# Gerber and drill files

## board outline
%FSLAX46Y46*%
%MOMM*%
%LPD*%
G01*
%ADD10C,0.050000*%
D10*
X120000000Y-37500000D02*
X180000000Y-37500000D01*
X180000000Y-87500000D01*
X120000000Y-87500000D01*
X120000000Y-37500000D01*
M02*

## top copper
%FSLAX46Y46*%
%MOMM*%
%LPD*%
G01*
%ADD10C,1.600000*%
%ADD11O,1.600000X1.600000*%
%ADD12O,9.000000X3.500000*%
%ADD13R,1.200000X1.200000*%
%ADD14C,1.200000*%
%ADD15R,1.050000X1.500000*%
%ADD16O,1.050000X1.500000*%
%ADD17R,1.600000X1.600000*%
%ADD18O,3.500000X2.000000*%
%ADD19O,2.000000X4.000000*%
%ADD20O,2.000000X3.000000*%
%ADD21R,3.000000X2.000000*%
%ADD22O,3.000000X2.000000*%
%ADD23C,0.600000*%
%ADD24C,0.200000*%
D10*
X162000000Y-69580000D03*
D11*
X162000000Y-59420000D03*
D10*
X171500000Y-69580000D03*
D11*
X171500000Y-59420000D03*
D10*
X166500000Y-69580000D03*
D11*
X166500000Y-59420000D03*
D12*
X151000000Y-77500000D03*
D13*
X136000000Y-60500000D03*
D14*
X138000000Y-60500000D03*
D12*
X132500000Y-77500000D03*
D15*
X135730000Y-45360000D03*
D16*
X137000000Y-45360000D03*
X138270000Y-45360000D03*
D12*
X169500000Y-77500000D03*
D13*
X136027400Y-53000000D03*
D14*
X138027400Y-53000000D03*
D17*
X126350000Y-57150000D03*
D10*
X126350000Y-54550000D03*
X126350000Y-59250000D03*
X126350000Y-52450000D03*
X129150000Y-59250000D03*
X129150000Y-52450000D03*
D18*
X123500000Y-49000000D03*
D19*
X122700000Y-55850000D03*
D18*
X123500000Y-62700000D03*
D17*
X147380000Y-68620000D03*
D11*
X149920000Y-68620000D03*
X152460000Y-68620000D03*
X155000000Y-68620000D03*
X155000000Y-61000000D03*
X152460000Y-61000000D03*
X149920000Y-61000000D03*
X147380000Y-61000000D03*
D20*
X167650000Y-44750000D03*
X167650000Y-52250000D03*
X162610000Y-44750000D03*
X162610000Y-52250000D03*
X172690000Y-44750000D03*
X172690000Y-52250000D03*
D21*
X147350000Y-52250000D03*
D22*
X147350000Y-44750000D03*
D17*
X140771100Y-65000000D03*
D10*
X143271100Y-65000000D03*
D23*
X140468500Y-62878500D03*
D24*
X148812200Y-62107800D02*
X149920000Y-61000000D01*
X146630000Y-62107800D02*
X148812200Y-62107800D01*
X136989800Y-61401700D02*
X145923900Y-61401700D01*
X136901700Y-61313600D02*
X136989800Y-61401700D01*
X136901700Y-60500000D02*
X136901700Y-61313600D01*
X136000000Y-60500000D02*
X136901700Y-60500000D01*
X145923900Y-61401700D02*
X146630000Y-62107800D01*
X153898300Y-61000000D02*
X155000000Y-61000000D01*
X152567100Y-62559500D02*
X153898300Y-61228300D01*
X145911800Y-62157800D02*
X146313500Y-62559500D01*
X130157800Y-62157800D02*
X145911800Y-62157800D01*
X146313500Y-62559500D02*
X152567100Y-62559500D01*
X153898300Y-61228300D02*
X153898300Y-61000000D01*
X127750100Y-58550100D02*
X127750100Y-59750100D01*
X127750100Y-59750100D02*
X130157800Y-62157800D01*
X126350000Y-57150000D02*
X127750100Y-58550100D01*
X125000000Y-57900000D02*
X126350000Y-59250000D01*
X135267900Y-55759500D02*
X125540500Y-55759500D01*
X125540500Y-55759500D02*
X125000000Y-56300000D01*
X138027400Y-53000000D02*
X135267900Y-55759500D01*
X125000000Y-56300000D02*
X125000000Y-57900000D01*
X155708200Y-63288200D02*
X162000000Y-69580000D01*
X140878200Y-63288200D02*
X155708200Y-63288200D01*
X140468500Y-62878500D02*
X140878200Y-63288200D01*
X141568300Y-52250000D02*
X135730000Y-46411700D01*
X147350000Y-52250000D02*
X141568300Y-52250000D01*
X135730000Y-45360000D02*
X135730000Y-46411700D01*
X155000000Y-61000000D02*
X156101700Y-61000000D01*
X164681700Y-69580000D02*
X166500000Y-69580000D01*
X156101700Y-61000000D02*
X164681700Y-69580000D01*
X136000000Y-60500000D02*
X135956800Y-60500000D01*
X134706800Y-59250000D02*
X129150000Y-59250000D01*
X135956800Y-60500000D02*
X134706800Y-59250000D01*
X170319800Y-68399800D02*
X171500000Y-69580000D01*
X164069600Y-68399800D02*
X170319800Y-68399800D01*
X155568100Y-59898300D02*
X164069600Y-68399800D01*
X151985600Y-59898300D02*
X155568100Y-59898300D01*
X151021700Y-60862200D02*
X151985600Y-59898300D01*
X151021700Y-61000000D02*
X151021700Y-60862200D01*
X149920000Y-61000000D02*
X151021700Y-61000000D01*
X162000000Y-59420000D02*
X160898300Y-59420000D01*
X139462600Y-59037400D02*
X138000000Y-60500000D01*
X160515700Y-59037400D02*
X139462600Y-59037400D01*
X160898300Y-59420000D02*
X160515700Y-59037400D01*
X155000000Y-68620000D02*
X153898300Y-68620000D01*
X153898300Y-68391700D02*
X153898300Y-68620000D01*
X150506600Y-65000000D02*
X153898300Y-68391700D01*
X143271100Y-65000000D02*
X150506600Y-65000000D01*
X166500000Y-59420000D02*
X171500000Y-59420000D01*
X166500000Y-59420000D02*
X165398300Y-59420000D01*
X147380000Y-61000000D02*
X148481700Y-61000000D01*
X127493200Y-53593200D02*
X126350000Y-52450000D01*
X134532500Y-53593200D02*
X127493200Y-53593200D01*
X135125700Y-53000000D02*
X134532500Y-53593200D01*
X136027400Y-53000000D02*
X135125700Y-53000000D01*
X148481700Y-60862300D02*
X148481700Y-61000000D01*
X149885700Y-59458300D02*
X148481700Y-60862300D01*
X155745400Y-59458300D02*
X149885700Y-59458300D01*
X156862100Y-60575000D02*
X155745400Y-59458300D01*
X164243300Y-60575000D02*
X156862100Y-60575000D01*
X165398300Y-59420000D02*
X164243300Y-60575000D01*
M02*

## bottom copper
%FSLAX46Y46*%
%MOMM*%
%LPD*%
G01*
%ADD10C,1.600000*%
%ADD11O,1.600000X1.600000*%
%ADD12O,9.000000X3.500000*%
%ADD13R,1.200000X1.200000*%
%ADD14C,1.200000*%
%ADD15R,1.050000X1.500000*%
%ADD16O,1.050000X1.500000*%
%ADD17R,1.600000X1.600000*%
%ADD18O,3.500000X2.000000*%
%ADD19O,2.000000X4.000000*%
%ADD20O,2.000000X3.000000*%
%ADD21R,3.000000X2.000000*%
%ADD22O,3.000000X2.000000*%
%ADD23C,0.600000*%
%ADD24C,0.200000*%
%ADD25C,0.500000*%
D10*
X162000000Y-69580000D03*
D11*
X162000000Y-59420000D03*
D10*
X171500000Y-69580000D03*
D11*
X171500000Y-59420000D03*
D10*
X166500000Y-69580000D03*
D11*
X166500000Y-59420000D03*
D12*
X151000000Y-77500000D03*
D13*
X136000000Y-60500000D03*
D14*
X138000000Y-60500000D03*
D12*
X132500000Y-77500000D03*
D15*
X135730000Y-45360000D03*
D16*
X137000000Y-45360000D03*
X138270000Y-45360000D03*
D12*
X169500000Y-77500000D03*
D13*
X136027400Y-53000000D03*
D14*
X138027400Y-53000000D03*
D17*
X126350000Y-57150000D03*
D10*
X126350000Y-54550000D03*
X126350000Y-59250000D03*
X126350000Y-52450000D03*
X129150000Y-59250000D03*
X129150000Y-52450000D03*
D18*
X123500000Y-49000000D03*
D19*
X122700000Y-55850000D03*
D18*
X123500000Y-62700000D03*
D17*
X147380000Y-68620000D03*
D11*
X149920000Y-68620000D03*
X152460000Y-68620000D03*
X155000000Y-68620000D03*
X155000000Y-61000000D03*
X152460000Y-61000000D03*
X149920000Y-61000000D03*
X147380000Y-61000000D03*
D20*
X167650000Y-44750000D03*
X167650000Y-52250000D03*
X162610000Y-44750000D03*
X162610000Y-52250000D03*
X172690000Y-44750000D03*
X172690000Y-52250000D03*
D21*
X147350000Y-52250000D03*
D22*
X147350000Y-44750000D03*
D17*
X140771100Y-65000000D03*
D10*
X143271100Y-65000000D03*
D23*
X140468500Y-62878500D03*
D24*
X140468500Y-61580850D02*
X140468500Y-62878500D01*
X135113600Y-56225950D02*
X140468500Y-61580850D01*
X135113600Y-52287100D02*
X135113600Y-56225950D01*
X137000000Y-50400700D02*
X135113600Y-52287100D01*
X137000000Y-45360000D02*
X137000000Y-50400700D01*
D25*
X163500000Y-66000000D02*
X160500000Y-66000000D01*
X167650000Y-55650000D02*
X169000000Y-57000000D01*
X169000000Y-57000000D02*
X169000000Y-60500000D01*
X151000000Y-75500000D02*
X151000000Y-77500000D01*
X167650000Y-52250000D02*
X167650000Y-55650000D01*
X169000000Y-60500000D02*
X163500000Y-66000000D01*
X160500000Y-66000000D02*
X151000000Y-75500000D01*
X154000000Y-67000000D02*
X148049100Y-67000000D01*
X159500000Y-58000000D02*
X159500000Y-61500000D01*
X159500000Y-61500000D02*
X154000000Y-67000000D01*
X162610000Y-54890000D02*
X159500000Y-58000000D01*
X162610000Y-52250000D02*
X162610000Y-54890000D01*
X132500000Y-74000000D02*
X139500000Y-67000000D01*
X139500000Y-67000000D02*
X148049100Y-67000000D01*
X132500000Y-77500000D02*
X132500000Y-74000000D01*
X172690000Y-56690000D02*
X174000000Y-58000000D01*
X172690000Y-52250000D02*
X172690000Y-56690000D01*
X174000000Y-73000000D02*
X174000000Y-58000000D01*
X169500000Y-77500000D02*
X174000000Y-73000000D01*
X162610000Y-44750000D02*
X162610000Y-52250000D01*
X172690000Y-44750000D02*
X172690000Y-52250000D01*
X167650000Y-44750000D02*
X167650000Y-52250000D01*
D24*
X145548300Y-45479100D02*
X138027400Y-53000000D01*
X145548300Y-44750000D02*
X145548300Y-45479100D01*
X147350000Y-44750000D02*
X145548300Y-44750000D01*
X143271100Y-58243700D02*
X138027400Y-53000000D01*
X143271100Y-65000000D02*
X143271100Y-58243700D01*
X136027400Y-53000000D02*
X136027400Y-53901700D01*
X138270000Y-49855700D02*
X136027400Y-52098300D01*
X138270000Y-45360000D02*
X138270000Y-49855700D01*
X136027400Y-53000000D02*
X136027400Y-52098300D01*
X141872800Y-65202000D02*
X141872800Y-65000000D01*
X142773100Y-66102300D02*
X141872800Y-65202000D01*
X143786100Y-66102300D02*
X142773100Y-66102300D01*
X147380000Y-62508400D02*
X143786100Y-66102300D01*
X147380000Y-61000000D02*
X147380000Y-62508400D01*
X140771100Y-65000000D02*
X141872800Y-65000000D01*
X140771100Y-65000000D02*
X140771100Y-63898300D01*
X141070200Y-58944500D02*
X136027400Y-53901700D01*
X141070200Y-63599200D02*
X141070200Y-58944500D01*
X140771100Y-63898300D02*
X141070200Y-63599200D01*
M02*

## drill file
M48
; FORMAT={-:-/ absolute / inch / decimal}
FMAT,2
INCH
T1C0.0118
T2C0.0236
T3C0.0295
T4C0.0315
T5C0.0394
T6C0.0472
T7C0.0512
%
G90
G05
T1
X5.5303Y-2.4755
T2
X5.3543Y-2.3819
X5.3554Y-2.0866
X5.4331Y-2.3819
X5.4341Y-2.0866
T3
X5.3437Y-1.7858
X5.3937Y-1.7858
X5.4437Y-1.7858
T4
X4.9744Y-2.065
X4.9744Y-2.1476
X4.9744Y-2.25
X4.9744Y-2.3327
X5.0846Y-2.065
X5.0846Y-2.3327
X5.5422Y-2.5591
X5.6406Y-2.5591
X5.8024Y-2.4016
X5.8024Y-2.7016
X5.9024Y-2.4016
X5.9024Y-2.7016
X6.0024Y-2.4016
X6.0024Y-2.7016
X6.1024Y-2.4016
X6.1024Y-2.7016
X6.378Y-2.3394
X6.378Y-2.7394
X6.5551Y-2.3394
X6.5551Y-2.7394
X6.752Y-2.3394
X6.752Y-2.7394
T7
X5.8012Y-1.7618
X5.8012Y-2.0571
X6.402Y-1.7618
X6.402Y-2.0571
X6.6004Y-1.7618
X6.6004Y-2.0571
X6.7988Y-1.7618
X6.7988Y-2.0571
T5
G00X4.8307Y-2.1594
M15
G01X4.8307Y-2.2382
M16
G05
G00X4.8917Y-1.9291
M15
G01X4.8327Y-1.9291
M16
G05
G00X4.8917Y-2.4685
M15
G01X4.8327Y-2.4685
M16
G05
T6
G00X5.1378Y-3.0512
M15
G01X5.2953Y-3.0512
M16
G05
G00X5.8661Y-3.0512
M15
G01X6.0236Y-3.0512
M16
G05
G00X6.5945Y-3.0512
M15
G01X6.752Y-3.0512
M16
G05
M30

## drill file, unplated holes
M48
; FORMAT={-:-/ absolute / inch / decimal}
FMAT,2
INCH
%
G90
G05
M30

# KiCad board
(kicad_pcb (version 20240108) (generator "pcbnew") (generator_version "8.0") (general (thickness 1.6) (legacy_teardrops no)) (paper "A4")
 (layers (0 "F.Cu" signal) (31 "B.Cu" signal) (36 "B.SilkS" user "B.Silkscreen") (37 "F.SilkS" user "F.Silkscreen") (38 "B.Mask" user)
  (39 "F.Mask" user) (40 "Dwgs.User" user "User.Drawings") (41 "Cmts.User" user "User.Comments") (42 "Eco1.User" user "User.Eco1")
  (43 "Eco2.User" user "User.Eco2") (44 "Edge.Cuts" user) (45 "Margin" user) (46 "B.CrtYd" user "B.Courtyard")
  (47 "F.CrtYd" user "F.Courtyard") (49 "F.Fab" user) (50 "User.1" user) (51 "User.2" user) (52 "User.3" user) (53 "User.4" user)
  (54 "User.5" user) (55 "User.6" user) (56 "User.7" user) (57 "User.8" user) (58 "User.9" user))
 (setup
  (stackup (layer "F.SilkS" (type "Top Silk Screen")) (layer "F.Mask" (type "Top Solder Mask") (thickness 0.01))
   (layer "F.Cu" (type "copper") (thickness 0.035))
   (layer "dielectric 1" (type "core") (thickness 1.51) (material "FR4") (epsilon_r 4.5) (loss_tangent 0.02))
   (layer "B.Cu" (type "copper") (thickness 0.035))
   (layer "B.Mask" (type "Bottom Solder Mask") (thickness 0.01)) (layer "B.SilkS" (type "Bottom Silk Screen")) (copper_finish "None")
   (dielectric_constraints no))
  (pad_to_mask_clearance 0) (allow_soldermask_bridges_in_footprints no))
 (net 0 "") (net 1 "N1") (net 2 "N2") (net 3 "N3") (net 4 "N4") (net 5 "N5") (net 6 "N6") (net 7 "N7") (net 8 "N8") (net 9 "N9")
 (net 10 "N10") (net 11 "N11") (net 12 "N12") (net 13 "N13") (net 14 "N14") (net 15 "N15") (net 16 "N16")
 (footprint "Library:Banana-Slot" (layer "F.Cu") (at 151 81.5)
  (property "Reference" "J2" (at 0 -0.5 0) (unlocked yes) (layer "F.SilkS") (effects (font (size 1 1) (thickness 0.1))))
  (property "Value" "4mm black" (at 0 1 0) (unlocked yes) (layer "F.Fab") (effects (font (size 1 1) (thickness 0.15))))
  (pad "1" thru_hole oval (at 0 -4) (size 9 3.5) (drill oval 5.2 1.2) (layers "*.Cu" "*.Mask") (remove_unused_layers no) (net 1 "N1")))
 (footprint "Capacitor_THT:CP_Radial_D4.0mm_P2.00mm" (layer "F.Cu") (at 136 60.5)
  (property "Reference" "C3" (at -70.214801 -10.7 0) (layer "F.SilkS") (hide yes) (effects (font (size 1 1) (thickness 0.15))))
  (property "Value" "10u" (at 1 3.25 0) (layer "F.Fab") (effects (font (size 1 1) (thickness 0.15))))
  (pad "1" thru_hole rect (at 0 0) (size 1.2 1.2) (drill 0.6) (layers "*.Cu" "*.Mask") (remove_unused_layers no) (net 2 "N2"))
  (pad "2" thru_hole circle (at 2 0) (size 1.2 1.2) (drill 0.6) (layers "*.Cu" "*.Mask") (remove_unused_layers no) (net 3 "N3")))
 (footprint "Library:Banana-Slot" (layer "F.Cu") (at 132.5 81.5)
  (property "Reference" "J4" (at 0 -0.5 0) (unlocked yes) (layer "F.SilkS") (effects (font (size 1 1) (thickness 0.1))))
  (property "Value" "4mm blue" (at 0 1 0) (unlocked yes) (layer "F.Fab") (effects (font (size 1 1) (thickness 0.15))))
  (pad "1" thru_hole oval (at 0 -4) (size 9 3.5) (drill oval 5.2 1.2) (layers "*.Cu" "*.Mask") (remove_unused_layers no) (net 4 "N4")))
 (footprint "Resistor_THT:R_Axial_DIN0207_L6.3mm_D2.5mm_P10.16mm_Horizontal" (layer "F.Cu") (at 171.5 69.58 90)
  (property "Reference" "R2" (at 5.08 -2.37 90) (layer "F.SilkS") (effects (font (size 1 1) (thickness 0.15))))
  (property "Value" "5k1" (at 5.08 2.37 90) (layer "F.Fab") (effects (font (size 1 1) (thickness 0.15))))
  (pad "1" thru_hole circle (at 0 0 90) (size 1.6 1.6) (drill 0.8) (layers "*.Cu" "*.Mask") (remove_unused_layers no) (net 2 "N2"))
  (pad "2" thru_hole oval (at 10.16 0 90) (size 1.6 1.6) (drill 0.8) (layers "*.Cu" "*.Mask") (remove_unused_layers no) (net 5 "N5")))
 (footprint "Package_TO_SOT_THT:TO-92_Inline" (layer "F.Cu") (at 135.73 45.36)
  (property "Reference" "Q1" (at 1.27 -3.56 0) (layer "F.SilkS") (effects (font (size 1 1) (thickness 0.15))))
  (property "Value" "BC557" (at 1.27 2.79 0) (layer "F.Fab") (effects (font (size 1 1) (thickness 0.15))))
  (pad "1" thru_hole rect (at 0 0) (size 1.05 1.5) (drill 0.75) (layers "*.Cu" "*.Mask") (remove_unused_layers no) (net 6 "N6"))
  (pad "2" thru_hole oval (at 1.27 0) (size 1.05 1.5) (drill 0.75) (layers "*.Cu" "*.Mask") (remove_unused_layers no) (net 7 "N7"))
  (pad "3" thru_hole oval (at 2.54 0) (size 1.05 1.5) (drill 0.75) (layers "*.Cu" "*.Mask") (remove_unused_layers no) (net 5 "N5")))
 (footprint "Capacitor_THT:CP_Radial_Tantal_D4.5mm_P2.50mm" (layer "F.Cu") (at 140.7711 65)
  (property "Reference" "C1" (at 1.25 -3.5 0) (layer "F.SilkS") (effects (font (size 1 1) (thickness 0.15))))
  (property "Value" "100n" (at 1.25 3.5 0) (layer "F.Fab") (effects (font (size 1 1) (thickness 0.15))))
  (pad "1" thru_hole rect (at 0 0) (size 1.6 1.6) (drill 0.8) (layers "*.Cu" "*.Mask") (remove_unused_layers no) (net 5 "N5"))
  (pad "2" thru_hole circle (at 2.5 0) (size 1.6 1.6) (drill 0.8) (layers "*.Cu" "*.Mask") (remove_unused_layers no) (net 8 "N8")))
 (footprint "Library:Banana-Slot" (layer "F.Cu") (at 169.5 81.5)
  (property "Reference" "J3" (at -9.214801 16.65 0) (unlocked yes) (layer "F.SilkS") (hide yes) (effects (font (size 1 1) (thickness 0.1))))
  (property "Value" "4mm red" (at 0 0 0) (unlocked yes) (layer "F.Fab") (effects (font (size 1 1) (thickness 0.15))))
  (pad "1" thru_hole oval (at 0 -4) (size 9 3.5) (drill oval 5.2 1.2) (layers "*.Cu" "*.Mask") (remove_unused_layers no) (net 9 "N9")))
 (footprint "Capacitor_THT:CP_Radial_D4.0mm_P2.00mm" (layer "F.Cu") (at 136.0274 53)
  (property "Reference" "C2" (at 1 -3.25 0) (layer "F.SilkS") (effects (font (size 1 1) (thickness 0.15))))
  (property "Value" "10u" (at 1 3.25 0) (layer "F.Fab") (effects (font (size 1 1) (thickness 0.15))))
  (pad "1" thru_hole rect (at 0 0) (size 1.2 1.2) (drill 0.6) (layers "*.Cu" "*.Mask") (remove_unused_layers no) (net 5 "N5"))
  (pad "2" thru_hole circle (at 2 0) (size 1.2 1.2) (drill 0.6) (layers "*.Cu" "*.Mask") (remove_unused_layers no) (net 8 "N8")))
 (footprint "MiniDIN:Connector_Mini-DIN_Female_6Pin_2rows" (layer "F.Cu") (at 126.35 57.15 -90)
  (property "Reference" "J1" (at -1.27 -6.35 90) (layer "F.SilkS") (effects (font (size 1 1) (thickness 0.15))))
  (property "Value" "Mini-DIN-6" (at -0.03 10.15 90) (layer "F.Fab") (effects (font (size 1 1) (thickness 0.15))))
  (pad "1" thru_hole rect (at 0 0 270) (size 1.6 1.6) (drill 0.8) (layers "*.Cu" "*.Mask") (remove_unused_layers no) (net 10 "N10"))
  (pad "2" thru_hole circle (at -2.6 0 270) (size 1.6 1.6) (drill 0.8) (layers "*.Cu" "*.Mask") (remove_unused_layers no) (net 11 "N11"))
  (pad "3" thru_hole circle (at 2.1 0 270) (size 1.6 1.6) (drill 0.8) (layers "*.Cu" "*.Mask") (remove_unused_layers no) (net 8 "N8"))
  (pad "4" thru_hole circle (at -4.7 0 270) (size 1.6 1.6) (drill 0.8) (layers "*.Cu" "*.Mask") (remove_unused_layers no) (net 5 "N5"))
  (pad "5" thru_hole circle (at 2.1 -2.8 270) (size 1.6 1.6) (drill 0.8) (layers "*.Cu" "*.Mask") (remove_unused_layers no) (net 2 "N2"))
  (pad "6" thru_hole circle (at -4.7 -2.8 270) (size 1.6 1.6) (drill 0.8) (layers "*.Cu" "*.Mask") (remove_unused_layers no) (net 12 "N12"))
  (pad "7" thru_hole oval (at -8.15 2.85 270) (size 2 3.5) (drill oval 1 2.5) (layers "*.Cu" "*.Mask") (remove_unused_layers no))
  (pad "7" thru_hole oval (at -1.3 3.65 270) (size 4 2) (drill oval 3 1) (layers "*.Cu" "*.Mask") (remove_unused_layers no))
  (pad "7" thru_hole oval (at 5.55 2.85 270) (size 2 3.5) (drill oval 1 2.5) (layers "*.Cu" "*.Mask") (remove_unused_layers no)))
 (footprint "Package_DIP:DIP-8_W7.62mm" (layer "F.Cu") (at 147.38 68.62 90)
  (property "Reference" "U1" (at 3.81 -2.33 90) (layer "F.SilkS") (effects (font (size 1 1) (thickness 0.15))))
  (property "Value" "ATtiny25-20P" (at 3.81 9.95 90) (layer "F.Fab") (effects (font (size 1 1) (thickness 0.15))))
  (pad "1" thru_hole rect (at 0 0 90) (size 1.6 1.6) (drill 0.8) (layers "*.Cu" "*.Mask") (remove_unused_layers no) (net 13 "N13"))
  (pad "2" thru_hole oval (at 0 2.54 90) (size 1.6 1.6) (drill 0.8) (layers "*.Cu" "*.Mask") (remove_unused_layers no) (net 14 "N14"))
  (pad "3" thru_hole oval (at 0 5.08 90) (size 1.6 1.6) (drill 0.8) (layers "*.Cu" "*.Mask") (remove_unused_layers no) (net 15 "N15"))
  (pad "4" thru_hole oval (at 0 7.62 90) (size 1.6 1.6) (drill 0.8) (layers "*.Cu" "*.Mask") (remove_unused_layers no) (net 8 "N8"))
  (pad "5" thru_hole oval (at 7.62 7.62 90) (size 1.6 1.6) (drill 0.8) (layers "*.Cu" "*.Mask") (remove_unused_layers no) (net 10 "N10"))
  (pad "6" thru_hole oval (at 7.62 5.08 90) (size 1.6 1.6) (drill 0.8) (layers "*.Cu" "*.Mask") (remove_unused_layers no) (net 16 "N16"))
  (pad "7" thru_hole oval (at 7.62 2.54 90) (size 1.6 1.6) (drill 0.8) (layers "*.Cu" "*.Mask") (remove_unused_layers no) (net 2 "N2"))
  (pad "8" thru_hole oval (at 7.62 0 90) (size 1.6 1.6) (drill 0.8) (layers "*.Cu" "*.Mask") (remove_unused_layers no) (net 5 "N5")))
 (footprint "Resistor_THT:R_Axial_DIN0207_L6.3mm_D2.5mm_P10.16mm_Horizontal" (layer "F.Cu") (at 162 69.58 90)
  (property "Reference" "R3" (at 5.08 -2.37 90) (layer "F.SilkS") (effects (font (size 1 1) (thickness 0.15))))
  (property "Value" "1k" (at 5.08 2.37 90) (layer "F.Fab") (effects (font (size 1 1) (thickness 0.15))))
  (pad "1" thru_hole circle (at 0 0 90) (size 1.6 1.6) (drill 0.8) (layers "*.Cu" "*.Mask") (remove_unused_layers no) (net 7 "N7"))
  (pad "2" thru_hole oval (at 10.16 0 90) (size 1.6 1.6) (drill 0.8) (layers "*.Cu" "*.Mask") (remove_unused_layers no) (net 3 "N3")))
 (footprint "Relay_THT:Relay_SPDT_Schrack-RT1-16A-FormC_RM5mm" (layer "F.Cu") (at 147.35 52.25)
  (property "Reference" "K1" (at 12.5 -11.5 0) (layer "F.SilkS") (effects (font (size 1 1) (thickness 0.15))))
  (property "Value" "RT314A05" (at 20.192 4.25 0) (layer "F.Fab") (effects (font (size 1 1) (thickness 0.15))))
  (pad "11" thru_hole oval (at 20.3 -7.5 180) (size 2 3) (drill 1.3) (layers "*.Cu" "*.Mask") (remove_unused_layers no) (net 1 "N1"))
  (pad "11" thru_hole oval (at 20.3 0 180) (size 2 3) (drill 1.3) (layers "*.Cu" "*.Mask") (remove_unused_layers no) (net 1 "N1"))
  (pad "12" thru_hole oval (at 15.26 -7.5 180) (size 2 3) (drill 1.3) (layers "*.Cu" "*.Mask") (remove_unused_layers no) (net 4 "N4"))
  (pad "12" thru_hole oval (at 15.26 0 180) (size 2 3) (drill 1.3) (layers "*.Cu" "*.Mask") (remove_unused_layers no) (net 4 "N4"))
  (pad "14" thru_hole oval (at 25.34 -7.5 180) (size 2 3) (drill 1.3) (layers "*.Cu" "*.Mask") (remove_unused_layers no) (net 9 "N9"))
  (pad "14" thru_hole oval (at 25.34 0 180) (size 2 3) (drill 1.3) (layers "*.Cu" "*.Mask") (remove_unused_layers no) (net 9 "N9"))
  (pad "A1" thru_hole rect (at 0 0 180) (size 3 2) (drill 1.3) (layers "*.Cu" "*.Mask") (remove_unused_layers no) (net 6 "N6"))
  (pad "A2" thru_hole oval (at 0 -7.5 180) (size 3 2) (drill 1.3) (layers "*.Cu" "*.Mask") (remove_unused_layers no) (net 8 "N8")))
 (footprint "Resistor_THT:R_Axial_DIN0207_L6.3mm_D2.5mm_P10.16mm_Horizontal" (layer "F.Cu") (at 166.5 69.58 90)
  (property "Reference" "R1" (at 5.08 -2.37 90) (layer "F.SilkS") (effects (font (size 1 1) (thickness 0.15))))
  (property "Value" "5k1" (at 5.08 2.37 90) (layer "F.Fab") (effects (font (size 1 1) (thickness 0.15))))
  (pad "1" thru_hole circle (at 0 0 90) (size 1.6 1.6) (drill 0.8) (layers "*.Cu" "*.Mask") (remove_unused_layers no) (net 10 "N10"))
  (pad "2" thru_hole oval (at 10.16 0 90) (size 1.6 1.6) (drill 0.8) (layers "*.Cu" "*.Mask") (remove_unused_layers no) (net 5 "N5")))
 (gr_rect (start 120 37.5) (end 180 87.5) (stroke (width 0.05) (type default)) (fill none) (layer "Edge.Cuts"))
 (segment (start 149.8857 59.4583) (end 148.4817 60.8623) (width 0.2) (layer "F.Cu") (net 5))
 (segment (start 136.0274 53) (end 135.1257 53) (width 0.2) (layer "F.Cu") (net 5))
 (segment (start 155.7454 59.4583) (end 149.8857 59.4583) (width 0.2) (layer "F.Cu") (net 5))
 (segment (start 134.5325 53.5932) (end 127.4932 53.5932) (width 0.2) (layer "F.Cu") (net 5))
 (segment (start 164.2433 60.575) (end 156.8621 60.575) (width 0.2) (layer "F.Cu") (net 5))
 (segment (start 148.4817 60.8623) (end 148.4817 61) (width 0.2) (layer "F.Cu") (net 5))
 (segment (start 165.3983 59.42) (end 164.2433 60.575) (width 0.2) (layer "F.Cu") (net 5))
 (segment (start 135.1257 53) (end 134.5325 53.5932) (width 0.2) (layer "F.Cu") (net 5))
 (segment (start 166.5 59.42) (end 171.5 59.42) (width 0.2) (layer "F.Cu") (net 5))
 (segment (start 147.38 61) (end 148.4817 61) (width 0.2) (layer "F.Cu") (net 5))
 (segment (start 156.8621 60.575) (end 155.7454 59.4583) (width 0.2) (layer "F.Cu") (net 5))
 (segment (start 166.5 59.42) (end 165.3983 59.42) (width 0.2) (layer "F.Cu") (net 5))
 (segment (start 127.4932 53.5932) (end 126.35 52.45) (width 0.2) (layer "F.Cu") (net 5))
 (segment (start 142.7731 66.1023) (end 141.8728 65.202) (width 0.2) (layer "B.Cu") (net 5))
 (segment (start 140.7711 63.8983) (end 141.0702 63.5992) (width 0.2) (layer "B.Cu") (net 5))
 (segment (start 138.27 49.8557) (end 136.0274 52.0983) (width 0.2) (layer "B.Cu") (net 5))
 (segment (start 136.0274 53) (end 136.0274 53.9017) (width 0.2) (layer "B.Cu") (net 5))
 (segment (start 141.8728 65.202) (end 141.8728 65) (width 0.2) (layer "B.Cu") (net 5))
 (segment (start 147.38 62.5084) (end 143.7861 66.1023) (width 0.2) (layer "B.Cu") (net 5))
 (segment (start 140.7711 65) (end 141.8728 65) (width 0.2) (layer "B.Cu") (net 5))
 (segment (start 143.7861 66.1023) (end 142.7731 66.1023) (width 0.2) (layer "B.Cu") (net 5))
 (segment (start 147.38 61) (end 147.38 62.5084) (width 0.2) (layer "B.Cu") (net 5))
 (segment (start 136.0274 53) (end 136.0274 52.0983) (width 0.2) (layer "B.Cu") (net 5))
 (segment (start 140.7711 65) (end 140.7711 63.8983) (width 0.2) (layer "B.Cu") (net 5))
 (segment (start 141.0702 58.9445) (end 136.0274 53.9017) (width 0.2) (layer "B.Cu") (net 5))
 (segment (start 138.27 45.36) (end 138.27 49.8557) (width 0.2) (layer "B.Cu") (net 5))
 (segment (start 141.0702 63.5992) (end 141.0702 58.9445) (width 0.2) (layer "B.Cu") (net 5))
 (segment (start 143.2711 65) (end 150.5066 65) (width 0.2) (layer "F.Cu") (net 8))
 (segment (start 150.5066 65) (end 153.8983 68.3917) (width 0.2) (layer "F.Cu") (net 8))
 (segment (start 153.8983 68.3917) (end 153.8983 68.62) (width 0.2) (layer "F.Cu") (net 8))
 (segment (start 138.0274 53) (end 135.2679 55.7595) (width 0.2) (layer "F.Cu") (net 8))
 (segment (start 135.2679 55.7595) (end 125.5405 55.7595) (width 0.2) (layer "F.Cu") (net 8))
 (segment (start 125.5405 55.7595) (end 125 56.3) (width 0.2) (layer "F.Cu") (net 8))
 (segment (start 155 68.62) (end 153.8983 68.62) (width 0.2) (layer "F.Cu") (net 8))
 (segment (start 125 56.3) (end 125 57.9) (width 0.2) (layer "F.Cu") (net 8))
 (segment (start 125 57.9) (end 126.35 59.25) (width 0.2) (layer "F.Cu") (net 8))
 (segment (start 143.2711 65) (end 143.2711 58.2437) (width 0.2) (layer "B.Cu") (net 8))
 (segment (start 145.5483 45.4791) (end 138.0274 53) (width 0.2) (layer "B.Cu") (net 8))
 (segment (start 147.35 44.75) (end 145.5483 44.75) (width 0.2) (layer "B.Cu") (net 8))
 (segment (start 145.5483 44.75) (end 145.5483 45.4791) (width 0.2) (layer "B.Cu") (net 8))
 (segment (start 143.2711 58.2437) (end 138.0274 53) (width 0.2) (layer "B.Cu") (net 8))
 (segment (start 139.4626 59.0374) (end 138 60.5) (width 0.2) (layer "F.Cu") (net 3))
 (segment (start 160.8983 59.42) (end 160.5157 59.0374) (width 0.2) (layer "F.Cu") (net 3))
 (segment (start 162 59.42) (end 160.8983 59.42) (width 0.2) (layer "F.Cu") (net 3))
 (segment (start 160.5157 59.0374) (end 139.4626 59.0374) (width 0.2) (layer "F.Cu") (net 3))
 (segment (start 151.9856 59.8983) (end 155.5681 59.8983) (width 0.2) (layer "F.Cu") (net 2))
 (segment (start 136.9017 61.3136) (end 136.9898 61.4017) (width 0.2) (layer "F.Cu") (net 2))
 (segment (start 151.0217 61) (end 151.0217 60.8622) (width 0.2) (layer "F.Cu") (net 2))
 (segment (start 136.9017 60.5) (end 136.9017 61.3136) (width 0.2) (layer "F.Cu") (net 2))
 (segment (start 155.5681 59.8983) (end 164.0696 68.3998) (width 0.2) (layer "F.Cu") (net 2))
 (segment (start 170.3198 68.3998) (end 171.5 69.58) (width 0.2) (layer "F.Cu") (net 2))
 (segment (start 135.9568 60.5) (end 134.7068 59.25) (width 0.2) (layer "F.Cu") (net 2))
 (segment (start 164.0696 68.3998) (end 170.3198 68.3998) (width 0.2) (layer "F.Cu") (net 2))
 (segment (start 145.9239 61.4017) (end 146.63 62.1078) (width 0.2) (layer "F.Cu") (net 2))
 (segment (start 136.9898 61.4017) (end 145.9239 61.4017) (width 0.2) (layer "F.Cu") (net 2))
 (segment (start 151.0217 60.8622) (end 151.9856 59.8983) (width 0.2) (layer "F.Cu") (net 2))
 (segment (start 136 60.5) (end 135.9568 60.5) (width 0.2) (layer "F.Cu") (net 2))
 (segment (start 149.92 61) (end 151.0217 61) (width 0.2) (layer "F.Cu") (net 2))
 (segment (start 146.63 62.1078) (end 148.8122 62.1078) (width 0.2) (layer "F.Cu") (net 2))
 (segment (start 136 60.5) (end 136.9017 60.5) (width 0.2) (layer "F.Cu") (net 2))
 (segment (start 148.8122 62.1078) (end 149.92 61) (width 0.2) (layer "F.Cu") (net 2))
 (segment (start 134.7068 59.25) (end 129.15 59.25) (width 0.2) (layer "F.Cu") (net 2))
 (segment (start 164.6817 69.58) (end 166.5 69.58) (width 0.2) (layer "F.Cu") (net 10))
 (segment (start 153.8983 61.2283) (end 153.8983 61) (width 0.2) (layer "F.Cu") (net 10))
 (segment (start 130.1578 62.1578) (end 145.9118 62.1578) (width 0.2) (layer "F.Cu") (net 10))
 (segment (start 153.8983 61) (end 155 61) (width 0.2) (layer "F.Cu") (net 10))
 (segment (start 152.5671 62.5595) (end 153.8983 61.2283) (width 0.2) (layer "F.Cu") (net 10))
 (segment (start 126.35 57.15) (end 127.7501 58.5501) (width 0.2) (layer "F.Cu") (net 10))
 (segment (start 155 61) (end 156.1017 61) (width 0.2) (layer "F.Cu") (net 10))
 (segment (start 127.7501 58.5501) (end 127.7501 59.7501) (width 0.2) (layer "F.Cu") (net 10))
 (segment (start 156.1017 61) (end 164.6817 69.58) (width 0.2) (layer "F.Cu") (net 10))
 (segment (start 146.3135 62.5595) (end 152.5671 62.5595) (width 0.2) (layer "F.Cu") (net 10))
 (segment (start 145.9118 62.1578) (end 146.3135 62.5595) (width 0.2) (layer "F.Cu") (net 10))
 (segment (start 127.7501 59.7501) (end 130.1578 62.1578) (width 0.2) (layer "F.Cu") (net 10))
 (segment (start 167.65 55.65) (end 169 57) (width 0.5) (layer "B.Cu") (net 1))
 (segment (start 167.65 44.75) (end 167.65 52.25) (width 0.5) (layer "B.Cu") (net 1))
 (segment (start 151 75.5) (end 151 77.5) (width 0.5) (layer "B.Cu") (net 1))
 (segment (start 169 57) (end 169 60.5) (width 0.5) (layer "B.Cu") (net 1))
 (segment (start 169 60.5) (end 163.5 66) (width 0.5) (layer "B.Cu") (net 1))
 (segment (start 167.65 52.25) (end 167.65 55.65) (width 0.5) (layer "B.Cu") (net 1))
 (segment (start 160.5 66) (end 151 75.5) (width 0.5) (layer "B.Cu") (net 1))
 (segment (start 163.5 66) (end 160.5 66) (width 0.5) (layer "B.Cu") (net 1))
 (segment (start 172.69 56.69) (end 174 58) (width 0.5) (layer "B.Cu") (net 9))
 (segment (start 172.69 52.25) (end 172.69 56.69) (width 0.5) (layer "B.Cu") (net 9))
 (segment (start 174 73) (end 174 58) (width 0.5) (layer "B.Cu") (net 9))
 (segment (start 172.69 44.75) (end 172.69 52.25) (width 0.5) (layer "B.Cu") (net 9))
 (segment (start 169.5 77.5) (end 174 73) (width 0.5) (layer "B.Cu") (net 9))
 (segment (start 139.5 67) (end 148.0491 67) (width 0.5) (layer "B.Cu") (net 4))
 (segment (start 154 67) (end 148.0491 67) (width 0.5) (layer "B.Cu") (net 4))
 (segment (start 162.61 44.75) (end 162.61 52.25) (width 0.5) (layer "B.Cu") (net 4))
 (segment (start 159.5 58) (end 159.5 61.5) (width 0.5) (layer "B.Cu") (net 4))
 (segment (start 132.5 77.5) (end 132.5 74) (width 0.5) (layer "B.Cu") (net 4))
 (segment (start 162.61 54.89) (end 159.5 58) (width 0.5) (layer "B.Cu") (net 4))
 (segment (start 132.5 74) (end 139.5 67) (width 0.5) (layer "B.Cu") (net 4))
 (segment (start 162.61 52.25) (end 162.61 54.89) (width 0.5) (layer "B.Cu") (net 4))
 (segment (start 159.5 61.5) (end 154 67) (width 0.5) (layer "B.Cu") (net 4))
 (segment (start 135.73 45.36) (end 135.73 46.4117) (width 0.2) (layer "F.Cu") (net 6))
 (segment (start 147.35 52.25) (end 141.5683 52.25) (width 0.2) (layer "F.Cu") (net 6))
 (segment (start 141.5683 52.25) (end 135.73 46.4117) (width 0.2) (layer "F.Cu") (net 6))
 (segment (start 155.7082 63.2882) (end 162 69.58) (width 0.2) (layer "F.Cu") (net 7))
 (segment (start 140.4685 62.8785) (end 140.8782 63.2882) (width 0.2) (layer "F.Cu") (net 7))
 (segment (start 140.8782 63.2882) (end 155.7082 63.2882) (width 0.2) (layer "F.Cu") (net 7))
 (via (at 140.4685 62.8785) (size 0.6) (drill 0.3) (layers "F.Cu" "B.Cu") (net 7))
 (segment (start 137 45.36) (end 137 50.4007) (width 0.2) (layer "B.Cu") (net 7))
 (segment (start 137 50.4007) (end 135.1136 52.2871) (width 0.2) (layer "B.Cu") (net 7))
 (segment (start 135.1136 56.22595) (end 140.4685 61.58085) (width 0.2) (layer "B.Cu") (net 7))
 (segment (start 140.4685 61.58085) (end 140.4685 62.8785) (width 0.2) (layer "B.Cu") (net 7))
 (segment (start 135.1136 52.2871) (end 135.1136 56.22595) (width 0.2) (layer "B.Cu") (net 7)))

